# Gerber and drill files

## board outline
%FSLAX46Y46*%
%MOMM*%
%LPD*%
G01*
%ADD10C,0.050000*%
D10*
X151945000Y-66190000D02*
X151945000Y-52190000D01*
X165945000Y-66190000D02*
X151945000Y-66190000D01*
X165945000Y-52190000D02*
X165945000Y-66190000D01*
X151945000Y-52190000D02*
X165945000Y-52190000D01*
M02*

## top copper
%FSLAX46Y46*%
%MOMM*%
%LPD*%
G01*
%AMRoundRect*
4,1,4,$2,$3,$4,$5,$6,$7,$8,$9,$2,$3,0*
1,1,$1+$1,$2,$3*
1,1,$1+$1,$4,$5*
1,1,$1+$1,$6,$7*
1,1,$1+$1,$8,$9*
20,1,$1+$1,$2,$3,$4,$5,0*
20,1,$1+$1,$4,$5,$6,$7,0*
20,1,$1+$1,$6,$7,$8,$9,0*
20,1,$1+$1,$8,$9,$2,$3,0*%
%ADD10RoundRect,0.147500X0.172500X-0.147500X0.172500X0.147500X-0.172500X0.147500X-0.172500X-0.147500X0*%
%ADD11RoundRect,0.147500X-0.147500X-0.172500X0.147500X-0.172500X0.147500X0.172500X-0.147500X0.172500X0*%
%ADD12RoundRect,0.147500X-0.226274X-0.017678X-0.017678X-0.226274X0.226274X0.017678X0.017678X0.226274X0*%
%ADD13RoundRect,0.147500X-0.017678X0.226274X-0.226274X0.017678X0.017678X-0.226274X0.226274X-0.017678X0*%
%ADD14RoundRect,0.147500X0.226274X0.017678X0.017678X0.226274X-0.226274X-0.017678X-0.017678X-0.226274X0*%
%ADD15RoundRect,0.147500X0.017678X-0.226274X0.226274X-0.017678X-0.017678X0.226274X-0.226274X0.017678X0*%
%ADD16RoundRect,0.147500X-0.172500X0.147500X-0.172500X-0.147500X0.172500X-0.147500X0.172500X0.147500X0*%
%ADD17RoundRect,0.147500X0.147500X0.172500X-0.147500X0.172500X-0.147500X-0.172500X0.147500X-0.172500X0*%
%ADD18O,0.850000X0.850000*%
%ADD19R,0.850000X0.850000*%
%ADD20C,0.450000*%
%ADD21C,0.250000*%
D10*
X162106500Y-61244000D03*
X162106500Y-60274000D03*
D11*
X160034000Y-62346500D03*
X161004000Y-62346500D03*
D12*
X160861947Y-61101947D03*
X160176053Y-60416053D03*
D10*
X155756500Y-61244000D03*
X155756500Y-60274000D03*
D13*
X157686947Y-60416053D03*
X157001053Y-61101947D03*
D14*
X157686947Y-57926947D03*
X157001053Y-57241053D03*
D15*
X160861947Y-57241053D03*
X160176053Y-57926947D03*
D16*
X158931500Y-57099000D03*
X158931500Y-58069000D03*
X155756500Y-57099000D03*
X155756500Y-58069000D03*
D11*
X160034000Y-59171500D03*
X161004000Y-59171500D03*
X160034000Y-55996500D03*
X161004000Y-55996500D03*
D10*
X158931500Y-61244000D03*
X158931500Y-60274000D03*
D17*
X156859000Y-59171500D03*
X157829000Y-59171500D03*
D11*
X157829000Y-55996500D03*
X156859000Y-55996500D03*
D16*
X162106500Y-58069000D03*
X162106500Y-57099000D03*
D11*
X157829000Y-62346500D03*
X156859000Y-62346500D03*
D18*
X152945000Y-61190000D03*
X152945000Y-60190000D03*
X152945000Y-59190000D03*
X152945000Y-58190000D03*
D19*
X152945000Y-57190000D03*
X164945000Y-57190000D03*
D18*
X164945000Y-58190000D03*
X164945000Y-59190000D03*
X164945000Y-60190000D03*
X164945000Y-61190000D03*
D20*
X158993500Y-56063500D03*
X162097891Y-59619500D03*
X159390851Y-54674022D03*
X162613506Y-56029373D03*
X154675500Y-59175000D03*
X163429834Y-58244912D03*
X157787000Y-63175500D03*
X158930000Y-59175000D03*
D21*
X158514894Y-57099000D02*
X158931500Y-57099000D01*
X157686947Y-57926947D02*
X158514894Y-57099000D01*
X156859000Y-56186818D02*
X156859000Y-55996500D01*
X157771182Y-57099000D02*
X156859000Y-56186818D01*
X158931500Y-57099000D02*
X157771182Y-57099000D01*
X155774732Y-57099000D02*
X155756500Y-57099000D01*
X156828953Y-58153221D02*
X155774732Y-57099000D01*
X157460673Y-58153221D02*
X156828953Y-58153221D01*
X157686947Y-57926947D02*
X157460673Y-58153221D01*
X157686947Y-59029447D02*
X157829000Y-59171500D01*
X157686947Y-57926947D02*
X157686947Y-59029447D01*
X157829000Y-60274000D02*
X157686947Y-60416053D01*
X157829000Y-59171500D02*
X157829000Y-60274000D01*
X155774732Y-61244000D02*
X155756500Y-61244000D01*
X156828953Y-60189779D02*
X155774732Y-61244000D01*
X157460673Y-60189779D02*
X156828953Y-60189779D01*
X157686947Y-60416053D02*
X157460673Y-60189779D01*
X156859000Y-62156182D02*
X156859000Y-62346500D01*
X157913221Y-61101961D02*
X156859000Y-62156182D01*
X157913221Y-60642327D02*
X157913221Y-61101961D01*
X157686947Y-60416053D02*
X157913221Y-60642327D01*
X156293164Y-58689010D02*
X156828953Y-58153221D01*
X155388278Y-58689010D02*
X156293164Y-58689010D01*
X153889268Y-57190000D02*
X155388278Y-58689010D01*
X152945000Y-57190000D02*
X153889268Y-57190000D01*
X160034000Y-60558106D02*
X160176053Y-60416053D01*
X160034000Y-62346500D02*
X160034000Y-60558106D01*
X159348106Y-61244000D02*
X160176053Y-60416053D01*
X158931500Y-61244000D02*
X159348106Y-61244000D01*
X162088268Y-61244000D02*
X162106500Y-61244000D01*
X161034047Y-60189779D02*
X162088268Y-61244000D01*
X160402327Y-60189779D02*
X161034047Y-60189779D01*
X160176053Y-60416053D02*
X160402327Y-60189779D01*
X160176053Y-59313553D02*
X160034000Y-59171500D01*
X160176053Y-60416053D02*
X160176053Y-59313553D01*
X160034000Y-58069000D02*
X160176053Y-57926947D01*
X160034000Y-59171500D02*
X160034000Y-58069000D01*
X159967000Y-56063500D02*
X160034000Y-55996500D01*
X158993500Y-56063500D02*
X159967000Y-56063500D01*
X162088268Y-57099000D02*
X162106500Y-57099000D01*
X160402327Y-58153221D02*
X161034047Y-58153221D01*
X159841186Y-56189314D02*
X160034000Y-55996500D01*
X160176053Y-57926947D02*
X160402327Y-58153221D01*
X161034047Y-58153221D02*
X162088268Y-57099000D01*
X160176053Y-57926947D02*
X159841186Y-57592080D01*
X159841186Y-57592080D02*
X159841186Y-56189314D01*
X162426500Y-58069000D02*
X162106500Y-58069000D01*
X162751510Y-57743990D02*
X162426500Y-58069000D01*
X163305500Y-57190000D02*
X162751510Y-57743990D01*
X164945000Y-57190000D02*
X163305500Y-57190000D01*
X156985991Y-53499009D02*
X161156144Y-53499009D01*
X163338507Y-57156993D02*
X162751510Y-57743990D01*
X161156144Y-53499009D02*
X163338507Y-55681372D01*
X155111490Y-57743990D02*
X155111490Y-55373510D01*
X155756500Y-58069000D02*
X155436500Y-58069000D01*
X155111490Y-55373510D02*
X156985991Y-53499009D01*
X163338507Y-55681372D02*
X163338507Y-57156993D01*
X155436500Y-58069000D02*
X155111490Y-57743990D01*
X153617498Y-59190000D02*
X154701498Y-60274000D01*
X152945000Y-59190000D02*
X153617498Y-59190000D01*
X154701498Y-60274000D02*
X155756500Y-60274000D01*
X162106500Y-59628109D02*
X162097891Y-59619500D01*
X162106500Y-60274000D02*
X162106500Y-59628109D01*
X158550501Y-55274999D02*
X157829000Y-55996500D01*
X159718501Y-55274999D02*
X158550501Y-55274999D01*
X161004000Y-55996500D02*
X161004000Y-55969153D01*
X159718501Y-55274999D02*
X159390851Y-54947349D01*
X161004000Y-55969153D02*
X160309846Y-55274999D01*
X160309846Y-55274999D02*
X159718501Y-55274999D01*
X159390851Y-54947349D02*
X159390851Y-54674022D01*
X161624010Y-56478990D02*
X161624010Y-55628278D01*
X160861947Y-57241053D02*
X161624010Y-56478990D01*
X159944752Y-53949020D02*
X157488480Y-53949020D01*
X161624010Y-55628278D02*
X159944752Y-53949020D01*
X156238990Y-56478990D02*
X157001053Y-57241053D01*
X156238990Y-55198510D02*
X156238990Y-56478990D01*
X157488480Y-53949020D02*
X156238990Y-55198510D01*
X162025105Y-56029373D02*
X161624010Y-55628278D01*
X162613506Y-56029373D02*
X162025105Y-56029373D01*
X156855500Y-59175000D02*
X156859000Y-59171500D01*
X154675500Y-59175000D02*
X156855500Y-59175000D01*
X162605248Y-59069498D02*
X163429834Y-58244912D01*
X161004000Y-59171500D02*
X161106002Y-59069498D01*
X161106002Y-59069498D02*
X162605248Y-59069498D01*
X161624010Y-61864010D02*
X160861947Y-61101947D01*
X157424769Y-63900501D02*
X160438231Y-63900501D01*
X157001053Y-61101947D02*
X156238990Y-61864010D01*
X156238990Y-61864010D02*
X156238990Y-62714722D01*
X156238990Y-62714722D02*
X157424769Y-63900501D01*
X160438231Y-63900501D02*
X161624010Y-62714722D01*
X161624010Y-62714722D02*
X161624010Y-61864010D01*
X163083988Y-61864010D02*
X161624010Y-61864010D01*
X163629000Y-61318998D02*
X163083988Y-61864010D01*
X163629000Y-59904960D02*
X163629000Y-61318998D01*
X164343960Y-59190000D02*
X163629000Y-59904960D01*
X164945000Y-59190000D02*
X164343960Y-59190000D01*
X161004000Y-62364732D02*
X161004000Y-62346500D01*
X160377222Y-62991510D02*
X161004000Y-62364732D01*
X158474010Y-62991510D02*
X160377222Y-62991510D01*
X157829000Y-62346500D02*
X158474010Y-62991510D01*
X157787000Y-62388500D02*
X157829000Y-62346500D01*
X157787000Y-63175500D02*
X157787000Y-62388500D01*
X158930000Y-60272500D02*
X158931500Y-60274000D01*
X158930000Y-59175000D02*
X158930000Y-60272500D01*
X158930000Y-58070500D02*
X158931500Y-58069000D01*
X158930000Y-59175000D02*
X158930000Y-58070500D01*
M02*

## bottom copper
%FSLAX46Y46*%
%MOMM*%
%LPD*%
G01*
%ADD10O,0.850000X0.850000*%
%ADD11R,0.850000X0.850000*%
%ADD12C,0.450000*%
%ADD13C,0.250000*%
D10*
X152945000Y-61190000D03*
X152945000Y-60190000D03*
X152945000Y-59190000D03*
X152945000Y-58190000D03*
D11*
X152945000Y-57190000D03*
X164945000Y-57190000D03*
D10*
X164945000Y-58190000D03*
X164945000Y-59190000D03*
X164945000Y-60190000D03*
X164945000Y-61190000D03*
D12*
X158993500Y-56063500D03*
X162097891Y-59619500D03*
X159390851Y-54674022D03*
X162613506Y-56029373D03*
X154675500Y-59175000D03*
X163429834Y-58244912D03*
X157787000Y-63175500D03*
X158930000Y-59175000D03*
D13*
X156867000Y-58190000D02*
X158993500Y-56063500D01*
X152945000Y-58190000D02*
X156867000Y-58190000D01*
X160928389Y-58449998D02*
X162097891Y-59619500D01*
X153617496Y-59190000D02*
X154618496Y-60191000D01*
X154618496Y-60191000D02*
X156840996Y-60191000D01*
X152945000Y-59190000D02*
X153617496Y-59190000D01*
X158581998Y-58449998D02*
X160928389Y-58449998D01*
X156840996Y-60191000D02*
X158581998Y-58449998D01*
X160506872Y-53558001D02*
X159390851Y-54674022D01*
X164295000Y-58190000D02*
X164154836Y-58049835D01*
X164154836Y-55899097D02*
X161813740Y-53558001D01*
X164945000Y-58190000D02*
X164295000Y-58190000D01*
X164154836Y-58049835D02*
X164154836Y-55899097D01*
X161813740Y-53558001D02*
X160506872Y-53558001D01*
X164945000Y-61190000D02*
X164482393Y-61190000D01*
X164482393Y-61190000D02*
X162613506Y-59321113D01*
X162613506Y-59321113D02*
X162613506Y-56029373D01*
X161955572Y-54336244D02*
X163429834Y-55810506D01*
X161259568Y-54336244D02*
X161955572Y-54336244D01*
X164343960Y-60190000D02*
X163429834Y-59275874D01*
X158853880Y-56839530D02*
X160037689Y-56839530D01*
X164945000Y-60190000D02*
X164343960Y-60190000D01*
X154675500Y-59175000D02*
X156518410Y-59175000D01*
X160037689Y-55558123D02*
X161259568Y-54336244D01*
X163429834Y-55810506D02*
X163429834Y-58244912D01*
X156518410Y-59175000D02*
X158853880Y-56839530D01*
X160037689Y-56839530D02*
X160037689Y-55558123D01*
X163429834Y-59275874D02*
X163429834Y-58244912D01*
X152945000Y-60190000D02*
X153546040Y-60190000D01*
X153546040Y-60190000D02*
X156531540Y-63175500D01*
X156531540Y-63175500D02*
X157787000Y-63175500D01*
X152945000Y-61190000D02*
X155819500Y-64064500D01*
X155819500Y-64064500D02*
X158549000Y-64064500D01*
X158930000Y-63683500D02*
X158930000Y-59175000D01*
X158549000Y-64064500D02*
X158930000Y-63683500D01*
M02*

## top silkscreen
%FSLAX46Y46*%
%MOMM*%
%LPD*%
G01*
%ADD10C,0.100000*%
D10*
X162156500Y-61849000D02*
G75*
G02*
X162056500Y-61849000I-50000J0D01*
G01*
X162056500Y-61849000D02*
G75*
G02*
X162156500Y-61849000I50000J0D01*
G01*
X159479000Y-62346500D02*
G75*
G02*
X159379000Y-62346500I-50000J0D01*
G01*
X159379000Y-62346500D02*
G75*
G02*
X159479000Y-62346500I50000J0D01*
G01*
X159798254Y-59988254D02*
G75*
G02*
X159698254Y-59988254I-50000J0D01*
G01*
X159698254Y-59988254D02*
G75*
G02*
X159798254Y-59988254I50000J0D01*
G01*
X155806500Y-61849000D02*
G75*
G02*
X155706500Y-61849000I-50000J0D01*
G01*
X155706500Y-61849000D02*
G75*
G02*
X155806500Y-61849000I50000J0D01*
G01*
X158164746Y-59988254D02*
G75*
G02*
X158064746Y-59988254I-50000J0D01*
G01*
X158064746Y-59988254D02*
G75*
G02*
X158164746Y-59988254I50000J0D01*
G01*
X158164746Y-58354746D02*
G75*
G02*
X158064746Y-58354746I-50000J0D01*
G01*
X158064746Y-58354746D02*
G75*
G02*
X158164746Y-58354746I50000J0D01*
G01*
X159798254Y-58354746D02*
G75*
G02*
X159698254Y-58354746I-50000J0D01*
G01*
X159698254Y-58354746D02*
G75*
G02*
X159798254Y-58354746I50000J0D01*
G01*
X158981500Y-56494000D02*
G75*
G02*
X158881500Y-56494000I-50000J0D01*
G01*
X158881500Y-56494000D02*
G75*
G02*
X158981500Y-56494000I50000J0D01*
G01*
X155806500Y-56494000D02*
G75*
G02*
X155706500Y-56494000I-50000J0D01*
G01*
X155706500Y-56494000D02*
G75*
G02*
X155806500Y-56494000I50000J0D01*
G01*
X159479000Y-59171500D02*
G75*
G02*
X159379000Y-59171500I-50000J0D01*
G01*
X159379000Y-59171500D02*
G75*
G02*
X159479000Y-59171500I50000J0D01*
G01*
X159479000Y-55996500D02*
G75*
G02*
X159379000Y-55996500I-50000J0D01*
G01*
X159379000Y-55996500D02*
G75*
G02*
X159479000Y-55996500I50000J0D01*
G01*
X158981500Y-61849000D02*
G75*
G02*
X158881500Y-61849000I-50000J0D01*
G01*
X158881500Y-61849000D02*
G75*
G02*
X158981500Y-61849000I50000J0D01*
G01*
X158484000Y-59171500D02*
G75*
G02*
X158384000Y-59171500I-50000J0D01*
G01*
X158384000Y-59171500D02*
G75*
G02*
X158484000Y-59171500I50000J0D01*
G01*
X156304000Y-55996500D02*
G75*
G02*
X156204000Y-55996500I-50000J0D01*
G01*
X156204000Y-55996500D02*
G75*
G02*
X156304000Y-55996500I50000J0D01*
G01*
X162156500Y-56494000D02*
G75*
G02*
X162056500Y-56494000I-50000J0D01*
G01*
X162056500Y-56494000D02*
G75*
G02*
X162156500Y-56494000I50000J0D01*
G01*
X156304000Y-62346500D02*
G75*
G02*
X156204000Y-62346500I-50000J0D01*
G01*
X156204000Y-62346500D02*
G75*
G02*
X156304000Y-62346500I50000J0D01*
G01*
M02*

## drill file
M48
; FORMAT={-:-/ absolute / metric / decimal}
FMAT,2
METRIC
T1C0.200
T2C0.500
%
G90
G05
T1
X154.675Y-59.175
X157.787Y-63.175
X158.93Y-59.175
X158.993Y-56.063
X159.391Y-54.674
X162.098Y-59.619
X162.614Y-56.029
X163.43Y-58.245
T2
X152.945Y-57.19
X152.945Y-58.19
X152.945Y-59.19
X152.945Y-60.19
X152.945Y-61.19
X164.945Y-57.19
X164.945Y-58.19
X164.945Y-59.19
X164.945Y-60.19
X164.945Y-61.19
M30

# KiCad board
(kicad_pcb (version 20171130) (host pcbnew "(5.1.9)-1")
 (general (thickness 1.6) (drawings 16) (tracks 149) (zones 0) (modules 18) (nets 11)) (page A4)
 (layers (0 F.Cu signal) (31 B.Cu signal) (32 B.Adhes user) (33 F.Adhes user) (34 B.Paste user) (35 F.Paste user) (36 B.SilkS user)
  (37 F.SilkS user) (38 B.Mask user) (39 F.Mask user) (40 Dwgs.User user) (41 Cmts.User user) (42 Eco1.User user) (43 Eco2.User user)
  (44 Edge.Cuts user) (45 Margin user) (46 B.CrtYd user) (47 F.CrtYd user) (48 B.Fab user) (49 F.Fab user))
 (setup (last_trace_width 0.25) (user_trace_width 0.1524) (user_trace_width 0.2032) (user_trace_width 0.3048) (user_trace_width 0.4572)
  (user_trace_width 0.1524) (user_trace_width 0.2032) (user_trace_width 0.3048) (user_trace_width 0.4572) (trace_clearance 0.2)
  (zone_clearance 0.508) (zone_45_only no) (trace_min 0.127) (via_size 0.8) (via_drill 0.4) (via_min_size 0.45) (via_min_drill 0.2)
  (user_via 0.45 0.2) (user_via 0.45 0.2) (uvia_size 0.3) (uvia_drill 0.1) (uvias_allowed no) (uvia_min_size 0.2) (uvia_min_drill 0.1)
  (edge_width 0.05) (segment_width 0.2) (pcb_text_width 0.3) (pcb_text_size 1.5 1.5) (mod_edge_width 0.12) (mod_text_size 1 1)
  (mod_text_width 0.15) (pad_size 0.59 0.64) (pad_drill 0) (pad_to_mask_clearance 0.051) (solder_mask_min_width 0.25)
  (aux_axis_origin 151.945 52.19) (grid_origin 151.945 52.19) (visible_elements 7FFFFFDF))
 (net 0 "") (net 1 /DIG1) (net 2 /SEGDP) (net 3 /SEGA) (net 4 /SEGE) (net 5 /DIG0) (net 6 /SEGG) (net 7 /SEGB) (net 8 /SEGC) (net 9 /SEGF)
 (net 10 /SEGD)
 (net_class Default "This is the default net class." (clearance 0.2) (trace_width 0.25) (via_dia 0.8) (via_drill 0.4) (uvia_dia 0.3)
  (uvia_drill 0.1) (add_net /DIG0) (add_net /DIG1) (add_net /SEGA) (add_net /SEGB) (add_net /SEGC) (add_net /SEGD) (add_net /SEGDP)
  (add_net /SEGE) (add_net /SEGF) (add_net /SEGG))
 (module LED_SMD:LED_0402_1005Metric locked (layer F.Cu) (at 162.1065 60.759 90)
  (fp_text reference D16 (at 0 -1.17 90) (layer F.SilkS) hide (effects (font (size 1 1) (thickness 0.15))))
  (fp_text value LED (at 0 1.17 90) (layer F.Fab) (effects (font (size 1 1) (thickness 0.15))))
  (fp_circle (center -1.09 0) (end -1.04 0) (layer F.SilkS) (width 0.1))
  (pad 1 smd roundrect (at -0.485 0 90) (size 0.59 0.64) (layers F.Cu F.Paste F.Mask) (roundrect_rratio 0.25) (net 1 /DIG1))
  (pad 2 smd roundrect (at 0.485 0 90) (size 0.59 0.64) (layers F.Cu F.Paste F.Mask) (roundrect_rratio 0.25) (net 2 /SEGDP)))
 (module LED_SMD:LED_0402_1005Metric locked (layer F.Cu) (at 160.519 62.3465)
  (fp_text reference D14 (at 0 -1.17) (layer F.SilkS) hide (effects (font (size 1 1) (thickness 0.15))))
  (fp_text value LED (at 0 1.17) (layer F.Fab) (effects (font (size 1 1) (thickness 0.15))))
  (fp_circle (center -1.09 0) (end -1.04 0) (layer F.SilkS) (width 0.1))
  (pad 1 smd roundrect (at -0.485 0) (size 0.59 0.64) (layers F.Cu F.Paste F.Mask) (roundrect_rratio 0.25) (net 1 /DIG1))
  (pad 2 smd roundrect (at 0.485 0) (size 0.59 0.64) (layers F.Cu F.Paste F.Mask) (roundrect_rratio 0.25) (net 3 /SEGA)))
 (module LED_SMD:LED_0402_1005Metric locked (layer F.Cu) (at 160.519 60.759 315)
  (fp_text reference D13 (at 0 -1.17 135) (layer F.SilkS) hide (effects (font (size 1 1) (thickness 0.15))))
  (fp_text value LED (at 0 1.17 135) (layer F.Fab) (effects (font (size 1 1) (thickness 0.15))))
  (fp_circle (center -1.09 0) (end -1.04 0) (layer F.SilkS) (width 0.1))
  (pad 2 smd roundrect (at 0.485 0 315) (size 0.59 0.64) (layers F.Cu F.Paste F.Mask) (roundrect_rratio 0.25) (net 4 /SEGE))
  (pad 1 smd roundrect (at -0.485 0 315) (size 0.59 0.64) (layers F.Cu F.Paste F.Mask) (roundrect_rratio 0.25) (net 1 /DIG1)))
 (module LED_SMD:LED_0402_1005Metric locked (layer F.Cu) (at 155.7565 60.759 90)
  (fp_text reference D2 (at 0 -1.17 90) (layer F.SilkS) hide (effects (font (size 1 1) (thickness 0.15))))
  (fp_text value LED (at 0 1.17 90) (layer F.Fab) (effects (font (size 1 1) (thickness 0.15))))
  (fp_circle (center -1.09 0) (end -1.04 0) (layer F.SilkS) (width 0.1))
  (pad 1 smd roundrect (at -0.485 0 90) (size 0.59 0.64) (layers F.Cu F.Paste F.Mask) (roundrect_rratio 0.25) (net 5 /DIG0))
  (pad 2 smd roundrect (at 0.485 0 90) (size 0.59 0.64) (layers F.Cu F.Paste F.Mask) (roundrect_rratio 0.25) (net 2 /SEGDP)))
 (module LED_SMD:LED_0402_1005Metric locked (layer F.Cu) (at 157.344 60.759 225)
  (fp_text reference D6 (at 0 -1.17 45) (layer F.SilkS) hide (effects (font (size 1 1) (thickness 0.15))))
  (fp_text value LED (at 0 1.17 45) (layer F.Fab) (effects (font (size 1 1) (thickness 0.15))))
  (fp_circle (center -1.09 0) (end -1.04 0) (layer F.SilkS) (width 0.1))
  (pad 1 smd roundrect (at -0.485 0 225) (size 0.59 0.64) (layers F.Cu F.Paste F.Mask) (roundrect_rratio 0.25) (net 5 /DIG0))
  (pad 2 smd roundrect (at 0.485 0 225) (size 0.59 0.64) (layers F.Cu F.Paste F.Mask) (roundrect_rratio 0.25) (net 4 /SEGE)))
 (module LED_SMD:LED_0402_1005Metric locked (layer F.Cu) (at 157.344 57.584 135)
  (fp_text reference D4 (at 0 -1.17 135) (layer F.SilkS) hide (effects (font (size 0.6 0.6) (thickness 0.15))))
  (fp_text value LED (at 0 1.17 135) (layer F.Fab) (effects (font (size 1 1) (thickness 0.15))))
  (fp_circle (center -1.09 0) (end -1.04 0) (layer F.SilkS) (width 0.1))
  (pad 1 smd roundrect (at -0.485 0 135) (size 0.59 0.64) (layers F.Cu F.Paste F.Mask) (roundrect_rratio 0.25) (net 5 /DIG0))
  (pad 2 smd roundrect (at 0.485 0 135) (size 0.59 0.64) (layers F.Cu F.Paste F.Mask) (roundrect_rratio 0.25) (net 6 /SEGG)))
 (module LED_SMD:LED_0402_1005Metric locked (layer F.Cu) (at 160.519 57.584 45)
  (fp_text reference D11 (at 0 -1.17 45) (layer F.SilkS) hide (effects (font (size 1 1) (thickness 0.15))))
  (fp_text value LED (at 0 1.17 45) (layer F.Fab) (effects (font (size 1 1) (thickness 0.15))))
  (fp_circle (center -1.09 0) (end -1.04 0) (layer F.SilkS) (width 0.1))
  (pad 2 smd roundrect (at 0.485 0 45) (size 0.59 0.64) (layers F.Cu F.Paste F.Mask) (roundrect_rratio 0.25) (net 6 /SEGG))
  (pad 1 smd roundrect (at -0.485 0 45) (size 0.59 0.64) (layers F.Cu F.Paste F.Mask) (roundrect_rratio 0.25) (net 1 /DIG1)))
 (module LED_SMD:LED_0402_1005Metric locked (layer F.Cu) (at 158.9315 57.584 270)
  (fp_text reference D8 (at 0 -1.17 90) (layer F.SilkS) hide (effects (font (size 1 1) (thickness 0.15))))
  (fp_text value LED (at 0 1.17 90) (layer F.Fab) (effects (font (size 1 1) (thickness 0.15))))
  (fp_circle (center -1.09 0) (end -1.04 0) (layer F.SilkS) (width 0.1))
  (pad 1 smd roundrect (at -0.485 0 270) (size 0.59 0.64) (layers F.Cu F.Paste F.Mask) (roundrect_rratio 0.25) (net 5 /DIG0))
  (pad 2 smd roundrect (at 0.485 0 270) (size 0.59 0.64) (layers F.Cu F.Paste F.Mask) (roundrect_rratio 0.25) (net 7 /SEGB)))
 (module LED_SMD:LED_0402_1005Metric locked (layer F.Cu) (at 155.7565 57.584 270)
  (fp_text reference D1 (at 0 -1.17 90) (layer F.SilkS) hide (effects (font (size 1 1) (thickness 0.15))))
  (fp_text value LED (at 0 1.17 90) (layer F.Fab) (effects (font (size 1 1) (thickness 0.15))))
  (fp_circle (center -1.09 0) (end -1.04 0) (layer F.SilkS) (width 0.1))
  (pad 1 smd roundrect (at -0.485 0 270) (size 0.59 0.64) (layers F.Cu F.Paste F.Mask) (roundrect_rratio 0.25) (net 5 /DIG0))
  (pad 2 smd roundrect (at 0.485 0 270) (size 0.59 0.64) (layers F.Cu F.Paste F.Mask) (roundrect_rratio 0.25) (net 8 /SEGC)))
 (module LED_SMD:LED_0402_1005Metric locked (layer F.Cu) (at 160.519 59.1715)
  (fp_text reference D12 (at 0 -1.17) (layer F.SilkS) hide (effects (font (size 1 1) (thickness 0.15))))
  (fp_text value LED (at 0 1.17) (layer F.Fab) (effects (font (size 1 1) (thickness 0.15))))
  (fp_circle (center -1.09 0) (end -1.04 0) (layer F.SilkS) (width 0.1))
  (pad 1 smd roundrect (at -0.485 0) (size 0.59 0.64) (layers F.Cu F.Paste F.Mask) (roundrect_rratio 0.25) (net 1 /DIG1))
  (pad 2 smd roundrect (at 0.485 0) (size 0.59 0.64) (layers F.Cu F.Paste F.Mask) (roundrect_rratio 0.25) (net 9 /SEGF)))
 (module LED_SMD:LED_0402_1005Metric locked (layer F.Cu) (at 160.519 55.9965)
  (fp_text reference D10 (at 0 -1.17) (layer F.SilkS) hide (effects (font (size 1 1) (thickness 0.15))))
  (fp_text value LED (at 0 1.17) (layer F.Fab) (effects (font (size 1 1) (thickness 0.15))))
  (fp_circle (center -1.09 0) (end -1.04 0) (layer F.SilkS) (width 0.1))
  (pad 1 smd roundrect (at -0.485 0) (size 0.59 0.64) (layers F.Cu F.Paste F.Mask) (roundrect_rratio 0.25) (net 1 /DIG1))
  (pad 2 smd roundrect (at 0.485 0) (size 0.59 0.64) (layers F.Cu F.Paste F.Mask) (roundrect_rratio 0.25) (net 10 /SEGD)))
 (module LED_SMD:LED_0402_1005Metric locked (layer F.Cu) (at 158.9315 60.759 90)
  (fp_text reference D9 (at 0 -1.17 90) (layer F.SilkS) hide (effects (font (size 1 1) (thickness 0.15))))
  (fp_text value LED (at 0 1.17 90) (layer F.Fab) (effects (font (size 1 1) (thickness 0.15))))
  (fp_circle (center -1.09 0) (end -1.04 0) (layer F.SilkS) (width 0.1))
  (pad 1 smd roundrect (at -0.485 0 90) (size 0.59 0.64) (layers F.Cu F.Paste F.Mask) (roundrect_rratio 0.25) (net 1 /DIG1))
  (pad 2 smd roundrect (at 0.485 0 90) (size 0.59 0.64) (layers F.Cu F.Paste F.Mask) (roundrect_rratio 0.25) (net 7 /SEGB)))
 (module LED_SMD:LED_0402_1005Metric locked (layer F.Cu) (at 157.344 59.1715 180)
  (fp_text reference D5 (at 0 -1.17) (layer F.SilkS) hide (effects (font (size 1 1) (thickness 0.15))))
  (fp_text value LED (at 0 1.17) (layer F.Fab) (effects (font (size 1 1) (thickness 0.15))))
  (fp_circle (center -1.09 0) (end -1.04 0) (layer F.SilkS) (width 0.1))
  (pad 2 smd roundrect (at 0.485 0 180) (size 0.59 0.64) (layers F.Cu F.Paste F.Mask) (roundrect_rratio 0.25) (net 9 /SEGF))
  (pad 1 smd roundrect (at -0.485 0 180) (size 0.59 0.64) (layers F.Cu F.Paste F.Mask) (roundrect_rratio 0.25) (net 5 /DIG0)))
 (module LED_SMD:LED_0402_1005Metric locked (layer F.Cu) (at 157.344 55.9965)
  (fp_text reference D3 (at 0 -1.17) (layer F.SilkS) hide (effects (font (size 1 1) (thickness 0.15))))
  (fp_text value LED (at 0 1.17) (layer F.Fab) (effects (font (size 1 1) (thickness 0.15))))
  (fp_circle (center -1.09 0) (end -1.04 0) (layer F.SilkS) (width 0.1))
  (pad 2 smd roundrect (at 0.485 0) (size 0.59 0.64) (layers F.Cu F.Paste F.Mask) (roundrect_rratio 0.25) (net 10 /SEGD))
  (pad 1 smd roundrect (at -0.485 0) (size 0.59 0.64) (layers F.Cu F.Paste F.Mask) (roundrect_rratio 0.25) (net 5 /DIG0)))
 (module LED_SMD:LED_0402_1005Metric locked (layer F.Cu) (at 162.1065 57.584 270)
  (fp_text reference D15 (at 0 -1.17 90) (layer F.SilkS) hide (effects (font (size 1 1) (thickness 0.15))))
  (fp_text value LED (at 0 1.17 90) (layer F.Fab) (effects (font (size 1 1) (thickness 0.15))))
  (fp_circle (center -1.09 0) (end -1.04 0) (layer F.SilkS) (width 0.1))
  (pad 2 smd roundrect (at 0.485 0 270) (size 0.59 0.64) (layers F.Cu F.Paste F.Mask) (roundrect_rratio 0.25) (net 8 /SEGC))
  (pad 1 smd roundrect (at -0.485 0 270) (size 0.59 0.64) (layers F.Cu F.Paste F.Mask) (roundrect_rratio 0.25) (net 1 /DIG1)))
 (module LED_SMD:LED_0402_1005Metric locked (layer F.Cu) (at 157.344 62.3465)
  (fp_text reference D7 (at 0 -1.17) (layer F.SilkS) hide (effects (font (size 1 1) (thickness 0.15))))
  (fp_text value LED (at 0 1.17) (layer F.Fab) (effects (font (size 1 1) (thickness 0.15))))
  (fp_circle (center -1.09 0) (end -1.04 0) (layer F.SilkS) (width 0.1))
  (pad 2 smd roundrect (at 0.485 0) (size 0.59 0.64) (layers F.Cu F.Paste F.Mask) (roundrect_rratio 0.25) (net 3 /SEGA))
  (pad 1 smd roundrect (at -0.485 0) (size 0.59 0.64) (layers F.Cu F.Paste F.Mask) (roundrect_rratio 0.25) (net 5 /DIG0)))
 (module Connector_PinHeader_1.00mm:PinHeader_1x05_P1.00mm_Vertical (layer B.Cu) (at 152.945 57.19 180)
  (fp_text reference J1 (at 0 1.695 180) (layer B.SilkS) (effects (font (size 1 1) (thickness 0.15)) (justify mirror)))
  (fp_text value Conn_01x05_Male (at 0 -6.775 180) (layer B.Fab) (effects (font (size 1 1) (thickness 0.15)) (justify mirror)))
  (pad 5 thru_hole oval (at 0 -4 180) (size 0.85 0.85) (drill 0.5) (layers *.Cu *.Mask) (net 7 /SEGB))
  (pad 4 thru_hole oval (at 0 -3 180) (size 0.85 0.85) (drill 0.5) (layers *.Cu *.Mask) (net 3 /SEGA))
  (pad 3 thru_hole oval (at 0 -2 180) (size 0.85 0.85) (drill 0.5) (layers *.Cu *.Mask) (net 2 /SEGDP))
  (pad 2 thru_hole oval (at 0 -1 180) (size 0.85 0.85) (drill 0.5) (layers *.Cu *.Mask) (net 1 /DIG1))
  (pad 1 thru_hole rect (at 0 0 180) (size 0.85 0.85) (drill 0.5) (layers *.Cu *.Mask) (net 5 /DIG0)))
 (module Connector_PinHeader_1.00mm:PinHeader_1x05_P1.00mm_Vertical (layer B.Cu) (at 164.945 57.19 180)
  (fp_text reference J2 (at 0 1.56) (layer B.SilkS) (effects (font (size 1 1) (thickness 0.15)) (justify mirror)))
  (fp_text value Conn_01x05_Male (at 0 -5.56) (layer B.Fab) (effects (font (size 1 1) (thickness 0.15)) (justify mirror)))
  (pad 1 thru_hole rect (at 0 0 180) (size 0.85 0.85) (drill 0.5) (layers *.Cu *.Mask) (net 8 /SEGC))
  (pad 2 thru_hole oval (at 0 -1 180) (size 0.85 0.85) (drill 0.5) (layers *.Cu *.Mask) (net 10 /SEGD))
  (pad 3 thru_hole oval (at 0 -2 180) (size 0.85 0.85) (drill 0.5) (layers *.Cu *.Mask) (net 4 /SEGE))
  (pad 4 thru_hole oval (at 0 -3 180) (size 0.85 0.85) (drill 0.5) (layers *.Cu *.Mask) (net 9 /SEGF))
  (pad 5 thru_hole oval (at 0 -4 180) (size 0.85 0.85) (drill 0.5) (layers *.Cu *.Mask) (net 6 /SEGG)))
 (gr_line (start 151.945 66.19) (end 151.945 52.19) (layer Edge.Cuts) (width 0.05))
 (gr_line (start 165.945 66.19) (end 151.945 66.19) (layer Edge.Cuts) (width 0.05))
 (gr_line (start 165.945 52.19) (end 165.945 66.19) (layer Edge.Cuts) (width 0.05))
 (gr_line (start 151.945 52.19) (end 165.945 52.19) (layer Edge.Cuts) (width 0.05))
 (segment (start 158.514894 57.099) (end 158.9315 57.099) (width 0.25) (layer F.Cu) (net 5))
 (segment (start 157.686947 57.926947) (end 158.514894 57.099) (width 0.25) (layer F.Cu) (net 5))
 (segment (start 156.859 56.186818) (end 156.859 55.9965) (width 0.25) (layer F.Cu) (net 5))
 (segment (start 157.771182 57.099) (end 156.859 56.186818) (width 0.25) (layer F.Cu) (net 5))
 (segment (start 158.9315 57.099) (end 157.771182 57.099) (width 0.25) (layer F.Cu) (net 5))
 (segment (start 155.774732 57.099) (end 155.7565 57.099) (width 0.25) (layer F.Cu) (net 5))
 (segment (start 156.828953 58.153221) (end 155.774732 57.099) (width 0.25) (layer F.Cu) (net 5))
 (segment (start 157.460673 58.153221) (end 156.828953 58.153221) (width 0.25) (layer F.Cu) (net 5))
 (segment (start 157.686947 57.926947) (end 157.460673 58.153221) (width 0.25) (layer F.Cu) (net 5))
 (segment (start 157.686947 59.029447) (end 157.829 59.1715) (width 0.25) (layer F.Cu) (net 5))
 (segment (start 157.686947 57.926947) (end 157.686947 59.029447) (width 0.25) (layer F.Cu) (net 5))
 (segment (start 157.829 60.274) (end 157.686947 60.416053) (width 0.25) (layer F.Cu) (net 5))
 (segment (start 157.829 59.1715) (end 157.829 60.274) (width 0.25) (layer F.Cu) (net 5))
 (segment (start 155.774732 61.244) (end 155.7565 61.244) (width 0.25) (layer F.Cu) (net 5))
 (segment (start 156.828953 60.189779) (end 155.774732 61.244) (width 0.25) (layer F.Cu) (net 5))
 (segment (start 157.460673 60.189779) (end 156.828953 60.189779) (width 0.25) (layer F.Cu) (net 5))
 (segment (start 157.686947 60.416053) (end 157.460673 60.189779) (width 0.25) (layer F.Cu) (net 5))
 (segment (start 156.859 62.156182) (end 156.859 62.3465) (width 0.25) (layer F.Cu) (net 5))
 (segment (start 157.913221 61.101961) (end 156.859 62.156182) (width 0.25) (layer F.Cu) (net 5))
 (segment (start 157.913221 60.642327) (end 157.913221 61.101961) (width 0.25) (layer F.Cu) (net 5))
 (segment (start 157.686947 60.416053) (end 157.913221 60.642327) (width 0.25) (layer F.Cu) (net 5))
 (segment (start 156.293164 58.68901) (end 156.828953 58.153221) (width 0.25) (layer F.Cu) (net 5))
 (segment (start 155.388278 58.68901) (end 156.293164 58.68901) (width 0.25) (layer F.Cu) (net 5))
 (segment (start 153.889268 57.19) (end 155.388278 58.68901) (width 0.25) (layer F.Cu) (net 5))
 (segment (start 152.945 57.19) (end 153.889268 57.19) (width 0.25) (layer F.Cu) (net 5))
 (segment (start 160.034 60.558106) (end 160.176053 60.416053) (width 0.25) (layer F.Cu) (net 1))
 (segment (start 160.034 62.3465) (end 160.034 60.558106) (width 0.25) (layer F.Cu) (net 1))
 (segment (start 159.348106 61.244) (end 160.176053 60.416053) (width 0.25) (layer F.Cu) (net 1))
 (segment (start 158.9315 61.244) (end 159.348106 61.244) (width 0.25) (layer F.Cu) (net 1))
 (segment (start 162.088268 61.244) (end 162.1065 61.244) (width 0.25) (layer F.Cu) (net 1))
 (segment (start 161.034047 60.189779) (end 162.088268 61.244) (width 0.25) (layer F.Cu) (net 1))
 (segment (start 160.402327 60.189779) (end 161.034047 60.189779) (width 0.25) (layer F.Cu) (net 1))
 (segment (start 160.176053 60.416053) (end 160.402327 60.189779) (width 0.25) (layer F.Cu) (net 1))
 (segment (start 160.176053 59.313553) (end 160.034 59.1715) (width 0.25) (layer F.Cu) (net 1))
 (segment (start 160.176053 60.416053) (end 160.176053 59.313553) (width 0.25) (layer F.Cu) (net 1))
 (segment (start 160.034 58.069) (end 160.176053 57.926947) (width 0.25) (layer F.Cu) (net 1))
 (segment (start 160.034 59.1715) (end 160.034 58.069) (width 0.25) (layer F.Cu) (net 1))
 (segment (start 156.867 58.19) (end 158.9935 56.0635) (width 0.25) (layer B.Cu) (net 1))
 (segment (start 152.945 58.19) (end 156.867 58.19) (width 0.25) (layer B.Cu) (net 1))
 (via (at 158.9935 56.0635) (size 0.45) (drill 0.2) (layers F.Cu B.Cu) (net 1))
 (segment (start 159.967 56.0635) (end 160.034 55.9965) (width 0.25) (layer F.Cu) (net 1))
 (segment (start 158.9935 56.0635) (end 159.967 56.0635) (width 0.25) (layer F.Cu) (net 1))
 (segment (start 162.088268 57.099) (end 162.1065 57.099) (width 0.25) (layer F.Cu) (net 1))
 (segment (start 160.402327 58.153221) (end 161.034047 58.153221) (width 0.25) (layer F.Cu) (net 1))
 (segment (start 159.841186 56.189314) (end 160.034 55.9965) (width 0.25) (layer F.Cu) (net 1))
 (segment (start 160.176053 57.926947) (end 160.402327 58.153221) (width 0.25) (layer F.Cu) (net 1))
 (segment (start 161.034047 58.153221) (end 162.088268 57.099) (width 0.25) (layer F.Cu) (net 1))
 (segment (start 160.176053 57.926947) (end 159.841186 57.59208) (width 0.25) (layer F.Cu) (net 1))
 (segment (start 159.841186 57.59208) (end 159.841186 56.189314) (width 0.25) (layer F.Cu) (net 1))
 (segment (start 162.4265 58.069) (end 162.1065 58.069) (width 0.25) (layer F.Cu) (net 8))
 (segment (start 162.75151 57.74399) (end 162.4265 58.069) (width 0.25) (layer F.Cu) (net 8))
 (segment (start 163.3055 57.19) (end 162.75151 57.74399) (width 0.25) (layer F.Cu) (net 8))
 (segment (start 164.945 57.19) (end 163.3055 57.19) (width 0.25) (layer F.Cu) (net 8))
 (segment (start 156.985991 53.499009) (end 161.156144 53.499009) (width 0.25) (layer F.Cu) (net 8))
 (segment (start 163.338507 57.156993) (end 162.75151 57.74399) (width 0.25) (layer F.Cu) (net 8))
 (segment (start 161.156144 53.499009) (end 163.338507 55.681372) (width 0.25) (layer F.Cu) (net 8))
 (segment (start 155.11149 57.74399) (end 155.11149 55.37351) (width 0.25) (layer F.Cu) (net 8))
 (segment (start 155.7565 58.069) (end 155.4365 58.069) (width 0.25) (layer F.Cu) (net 8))
 (segment (start 155.11149 55.37351) (end 156.985991 53.499009) (width 0.25) (layer F.Cu) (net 8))
 (segment (start 163.338507 55.681372) (end 163.338507 57.156993) (width 0.25) (layer F.Cu) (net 8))
 (segment (start 155.4365 58.069) (end 155.11149 57.74399) (width 0.25) (layer F.Cu) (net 8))
 (segment (start 153.617498 59.19) (end 154.701498 60.274) (width 0.25) (layer F.Cu) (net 2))
 (segment (start 152.945 59.19) (end 153.617498 59.19) (width 0.25) (layer F.Cu) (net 2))
 (segment (start 154.701498 60.274) (end 155.7565 60.274) (width 0.25) (layer F.Cu) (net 2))
 (segment (start 160.928389 58.449998) (end 162.097891 59.6195) (width 0.25) (layer B.Cu) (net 2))
 (segment (start 153.617496 59.19) (end 154.618496 60.191) (width 0.25) (layer B.Cu) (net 2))
 (segment (start 154.618496 60.191) (end 156.840996 60.191) (width 0.25) (layer B.Cu) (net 2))
 (segment (start 152.945 59.19) (end 153.617496 59.19) (width 0.25) (layer B.Cu) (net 2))
 (segment (start 158.581998 58.449998) (end 160.928389 58.449998) (width 0.25) (layer B.Cu) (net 2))
 (segment (start 162.1065 59.628109) (end 162.097891 59.6195) (width 0.25) (layer F.Cu) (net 2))
 (segment (start 162.1065 60.274) (end 162.1065 59.628109) (width 0.25) (layer F.Cu) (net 2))
 (via (at 162.097891 59.6195) (size 0.45) (drill 0.2) (layers F.Cu B.Cu) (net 2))
 (segment (start 156.840996 60.191) (end 158.581998 58.449998) (width 0.25) (layer B.Cu) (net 2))
 (segment (start 158.550501 55.274999) (end 157.829 55.9965) (width 0.25) (layer F.Cu) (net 10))
 (segment (start 159.718501 55.274999) (end 158.550501 55.274999) (width 0.25) (layer F.Cu) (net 10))
 (segment (start 160.506872 53.558001) (end 159.390851 54.674022) (width 0.25) (layer B.Cu) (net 10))
 (segment (start 161.004 55.9965) (end 161.004 55.969153) (width 0.25) (layer F.Cu) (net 10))
 (segment (start 159.718501 55.274999) (end 159.390851 54.947349) (width 0.25) (layer F.Cu) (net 10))
 (segment (start 164.295 58.19) (end 164.154836 58.049835) (width 0.25) (layer B.Cu) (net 10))
 (via (at 159.390851 54.674022) (size 0.45) (drill 0.2) (layers F.Cu B.Cu) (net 10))
 (segment (start 161.004 55.969153) (end 160.309846 55.274999) (width 0.25) (layer F.Cu) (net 10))
 (segment (start 164.154836 55.899097) (end 161.81374 53.558001) (width 0.25) (layer B.Cu) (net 10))
 (segment (start 160.309846 55.274999) (end 159.718501 55.274999) (width 0.25) (layer F.Cu) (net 10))
 (segment (start 164.945 58.19) (end 164.295 58.19) (width 0.25) (layer B.Cu) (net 10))
 (segment (start 164.154836 58.049835) (end 164.154836 55.899097) (width 0.25) (layer B.Cu) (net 10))
 (segment (start 161.81374 53.558001) (end 160.506872 53.558001) (width 0.25) (layer B.Cu) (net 10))
 (segment (start 159.390851 54.947349) (end 159.390851 54.674022) (width 0.25) (layer F.Cu) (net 10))
 (via (at 162.613506 56.029373) (size 0.45) (drill 0.2) (layers F.Cu B.Cu) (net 6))
 (segment (start 161.62401 56.47899) (end 161.62401 55.628278) (width 0.25) (layer F.Cu) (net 6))
 (segment (start 160.861947 57.241053) (end 161.62401 56.47899) (width 0.25) (layer F.Cu) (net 6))
 (segment (start 159.944752 53.94902) (end 157.48848 53.94902) (width 0.25) (layer F.Cu) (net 6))
 (segment (start 161.62401 55.628278) (end 159.944752 53.94902) (width 0.25) (layer F.Cu) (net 6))
 (segment (start 156.23899 56.47899) (end 157.001053 57.241053) (width 0.25) (layer F.Cu) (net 6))
 (segment (start 156.23899 55.19851) (end 156.23899 56.47899) (width 0.25) (layer F.Cu) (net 6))
 (segment (start 157.48848 53.94902) (end 156.23899 55.19851) (width 0.25) (layer F.Cu) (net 6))
 (segment (start 162.025105 56.029373) (end 161.62401 55.628278) (width 0.25) (layer F.Cu) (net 6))
 (segment (start 162.613506 56.029373) (end 162.025105 56.029373) (width 0.25) (layer F.Cu) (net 6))
 (segment (start 164.945 61.19) (end 164.482393 61.19) (width 0.25) (layer B.Cu) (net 6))
 (segment (start 164.482393 61.19) (end 162.613506 59.321113) (width 0.25) (layer B.Cu) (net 6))
 (segment (start 162.613506 59.321113) (end 162.613506 56.029373) (width 0.25) (layer B.Cu) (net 6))
 (via (at 154.6755 59.175) (size 0.45) (drill 0.2) (layers F.Cu B.Cu) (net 9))
 (segment (start 156.8555 59.175) (end 156.859 59.1715) (width 0.25) (layer F.Cu) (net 9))
 (segment (start 154.6755 59.175) (end 156.8555 59.175) (width 0.25) (layer F.Cu) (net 9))
 (segment (start 161.955572 54.336244) (end 163.429834 55.810506) (width 0.25) (layer B.Cu) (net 9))
 (segment (start 161.259568 54.336244) (end 161.955572 54.336244) (width 0.25) (layer B.Cu) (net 9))
 (segment (start 164.34396 60.19) (end 163.429834 59.275874) (width 0.25) (layer B.Cu) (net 9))
 (segment (start 158.85388 56.83953) (end 160.037689 56.83953) (width 0.25) (layer B.Cu) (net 9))
 (segment (start 164.945 60.19) (end 164.34396 60.19) (width 0.25) (layer B.Cu) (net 9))
 (segment (start 154.6755 59.175) (end 156.51841 59.175) (width 0.25) (layer B.Cu) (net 9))
 (segment (start 160.037689 55.558123) (end 161.259568 54.336244) (width 0.25) (layer B.Cu) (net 9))
 (segment (start 163.429834 55.810506) (end 163.429834 58.244912) (width 0.25) (layer B.Cu) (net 9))
 (segment (start 156.51841 59.175) (end 158.85388 56.83953) (width 0.25) (layer B.Cu) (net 9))
 (via (at 163.429834 58.244912) (size 0.45) (drill 0.2) (layers F.Cu B.Cu) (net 9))
 (segment (start 160.037689 56.83953) (end 160.037689 55.558123) (width 0.25) (layer B.Cu) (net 9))
 (segment (start 163.429834 59.275874) (end 163.429834 58.244912) (width 0.25) (layer B.Cu) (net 9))
 (segment (start 162.605248 59.069498) (end 163.429834 58.244912) (width 0.25) (layer F.Cu) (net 9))
 (segment (start 161.004 59.1715) (end 161.106002 59.069498) (width 0.25) (layer F.Cu) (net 9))
 (segment (start 161.106002 59.069498) (end 162.605248 59.069498) (width 0.25) (layer F.Cu) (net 9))
 (segment (start 161.62401 61.86401) (end 160.861947 61.101947) (width 0.25) (layer F.Cu) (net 4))
 (segment (start 157.424769 63.900501) (end 160.438231 63.900501) (width 0.25) (layer F.Cu) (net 4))
 (segment (start 157.001053 61.101947) (end 156.23899 61.86401) (width 0.25) (layer F.Cu) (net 4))
 (segment (start 156.23899 61.86401) (end 156.23899 62.714722) (width 0.25) (layer F.Cu) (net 4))
 (segment (start 156.23899 62.714722) (end 157.424769 63.900501) (width 0.25) (layer F.Cu) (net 4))
 (segment (start 160.438231 63.900501) (end 161.62401 62.714722) (width 0.25) (layer F.Cu) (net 4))
 (segment (start 161.62401 62.714722) (end 161.62401 61.86401) (width 0.25) (layer F.Cu) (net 4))
 (segment (start 163.083988 61.86401) (end 161.62401 61.86401) (width 0.25) (layer F.Cu) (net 4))
 (segment (start 163.629 61.318998) (end 163.083988 61.86401) (width 0.25) (layer F.Cu) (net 4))
 (segment (start 163.629 59.90496) (end 163.629 61.318998) (width 0.25) (layer F.Cu) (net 4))
 (segment (start 164.34396 59.19) (end 163.629 59.90496) (width 0.25) (layer F.Cu) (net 4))
 (segment (start 164.945 59.19) (end 164.34396 59.19) (width 0.25) (layer F.Cu) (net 4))
 (segment (start 161.004 62.364732) (end 161.004 62.3465) (width 0.25) (layer F.Cu) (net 3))
 (segment (start 160.377222 62.99151) (end 161.004 62.364732) (width 0.25) (layer F.Cu) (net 3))
 (segment (start 158.47401 62.99151) (end 160.377222 62.99151) (width 0.25) (layer F.Cu) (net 3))
 (segment (start 157.829 62.3465) (end 158.47401 62.99151) (width 0.25) (layer F.Cu) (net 3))
 (via (at 157.787 63.1755) (size 0.45) (drill 0.2) (layers F.Cu B.Cu) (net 3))
 (segment (start 157.787 62.3885) (end 157.829 62.3465) (width 0.25) (layer F.Cu) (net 3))
 (segment (start 157.787 63.1755) (end 157.787 62.3885) (width 0.25) (layer F.Cu) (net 3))
 (segment (start 152.945 60.19) (end 153.54604 60.19) (width 0.25) (layer B.Cu) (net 3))
 (segment (start 153.54604 60.19) (end 156.53154 63.1755) (width 0.25) (layer B.Cu) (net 3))
 (segment (start 156.53154 63.1755) (end 157.787 63.1755) (width 0.25) (layer B.Cu) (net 3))
 (segment (start 152.945 61.19) (end 155.8195 64.0645) (width 0.25) (layer B.Cu) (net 7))
 (segment (start 155.8195 64.0645) (end 158.549 64.0645) (width 0.25) (layer B.Cu) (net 7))
 (segment (start 158.93 63.6835) (end 158.93 59.175) (width 0.25) (layer B.Cu) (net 7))
 (via (at 158.93 59.175) (size 0.45) (drill 0.2) (layers F.Cu B.Cu) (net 7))
 (segment (start 158.549 64.0645) (end 158.93 63.6835) (width 0.25) (layer B.Cu) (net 7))
 (segment (start 158.93 60.2725) (end 158.9315 60.274) (width 0.25) (layer F.Cu) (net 7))
 (segment (start 158.93 59.175) (end 158.93 60.2725) (width 0.25) (layer F.Cu) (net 7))
 (segment (start 158.93 58.0705) (end 158.9315 58.069) (width 0.25) (layer F.Cu) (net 7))
 (segment (start 158.93 59.175) (end 158.93 58.0705) (width 0.25) (layer F.Cu) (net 7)))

